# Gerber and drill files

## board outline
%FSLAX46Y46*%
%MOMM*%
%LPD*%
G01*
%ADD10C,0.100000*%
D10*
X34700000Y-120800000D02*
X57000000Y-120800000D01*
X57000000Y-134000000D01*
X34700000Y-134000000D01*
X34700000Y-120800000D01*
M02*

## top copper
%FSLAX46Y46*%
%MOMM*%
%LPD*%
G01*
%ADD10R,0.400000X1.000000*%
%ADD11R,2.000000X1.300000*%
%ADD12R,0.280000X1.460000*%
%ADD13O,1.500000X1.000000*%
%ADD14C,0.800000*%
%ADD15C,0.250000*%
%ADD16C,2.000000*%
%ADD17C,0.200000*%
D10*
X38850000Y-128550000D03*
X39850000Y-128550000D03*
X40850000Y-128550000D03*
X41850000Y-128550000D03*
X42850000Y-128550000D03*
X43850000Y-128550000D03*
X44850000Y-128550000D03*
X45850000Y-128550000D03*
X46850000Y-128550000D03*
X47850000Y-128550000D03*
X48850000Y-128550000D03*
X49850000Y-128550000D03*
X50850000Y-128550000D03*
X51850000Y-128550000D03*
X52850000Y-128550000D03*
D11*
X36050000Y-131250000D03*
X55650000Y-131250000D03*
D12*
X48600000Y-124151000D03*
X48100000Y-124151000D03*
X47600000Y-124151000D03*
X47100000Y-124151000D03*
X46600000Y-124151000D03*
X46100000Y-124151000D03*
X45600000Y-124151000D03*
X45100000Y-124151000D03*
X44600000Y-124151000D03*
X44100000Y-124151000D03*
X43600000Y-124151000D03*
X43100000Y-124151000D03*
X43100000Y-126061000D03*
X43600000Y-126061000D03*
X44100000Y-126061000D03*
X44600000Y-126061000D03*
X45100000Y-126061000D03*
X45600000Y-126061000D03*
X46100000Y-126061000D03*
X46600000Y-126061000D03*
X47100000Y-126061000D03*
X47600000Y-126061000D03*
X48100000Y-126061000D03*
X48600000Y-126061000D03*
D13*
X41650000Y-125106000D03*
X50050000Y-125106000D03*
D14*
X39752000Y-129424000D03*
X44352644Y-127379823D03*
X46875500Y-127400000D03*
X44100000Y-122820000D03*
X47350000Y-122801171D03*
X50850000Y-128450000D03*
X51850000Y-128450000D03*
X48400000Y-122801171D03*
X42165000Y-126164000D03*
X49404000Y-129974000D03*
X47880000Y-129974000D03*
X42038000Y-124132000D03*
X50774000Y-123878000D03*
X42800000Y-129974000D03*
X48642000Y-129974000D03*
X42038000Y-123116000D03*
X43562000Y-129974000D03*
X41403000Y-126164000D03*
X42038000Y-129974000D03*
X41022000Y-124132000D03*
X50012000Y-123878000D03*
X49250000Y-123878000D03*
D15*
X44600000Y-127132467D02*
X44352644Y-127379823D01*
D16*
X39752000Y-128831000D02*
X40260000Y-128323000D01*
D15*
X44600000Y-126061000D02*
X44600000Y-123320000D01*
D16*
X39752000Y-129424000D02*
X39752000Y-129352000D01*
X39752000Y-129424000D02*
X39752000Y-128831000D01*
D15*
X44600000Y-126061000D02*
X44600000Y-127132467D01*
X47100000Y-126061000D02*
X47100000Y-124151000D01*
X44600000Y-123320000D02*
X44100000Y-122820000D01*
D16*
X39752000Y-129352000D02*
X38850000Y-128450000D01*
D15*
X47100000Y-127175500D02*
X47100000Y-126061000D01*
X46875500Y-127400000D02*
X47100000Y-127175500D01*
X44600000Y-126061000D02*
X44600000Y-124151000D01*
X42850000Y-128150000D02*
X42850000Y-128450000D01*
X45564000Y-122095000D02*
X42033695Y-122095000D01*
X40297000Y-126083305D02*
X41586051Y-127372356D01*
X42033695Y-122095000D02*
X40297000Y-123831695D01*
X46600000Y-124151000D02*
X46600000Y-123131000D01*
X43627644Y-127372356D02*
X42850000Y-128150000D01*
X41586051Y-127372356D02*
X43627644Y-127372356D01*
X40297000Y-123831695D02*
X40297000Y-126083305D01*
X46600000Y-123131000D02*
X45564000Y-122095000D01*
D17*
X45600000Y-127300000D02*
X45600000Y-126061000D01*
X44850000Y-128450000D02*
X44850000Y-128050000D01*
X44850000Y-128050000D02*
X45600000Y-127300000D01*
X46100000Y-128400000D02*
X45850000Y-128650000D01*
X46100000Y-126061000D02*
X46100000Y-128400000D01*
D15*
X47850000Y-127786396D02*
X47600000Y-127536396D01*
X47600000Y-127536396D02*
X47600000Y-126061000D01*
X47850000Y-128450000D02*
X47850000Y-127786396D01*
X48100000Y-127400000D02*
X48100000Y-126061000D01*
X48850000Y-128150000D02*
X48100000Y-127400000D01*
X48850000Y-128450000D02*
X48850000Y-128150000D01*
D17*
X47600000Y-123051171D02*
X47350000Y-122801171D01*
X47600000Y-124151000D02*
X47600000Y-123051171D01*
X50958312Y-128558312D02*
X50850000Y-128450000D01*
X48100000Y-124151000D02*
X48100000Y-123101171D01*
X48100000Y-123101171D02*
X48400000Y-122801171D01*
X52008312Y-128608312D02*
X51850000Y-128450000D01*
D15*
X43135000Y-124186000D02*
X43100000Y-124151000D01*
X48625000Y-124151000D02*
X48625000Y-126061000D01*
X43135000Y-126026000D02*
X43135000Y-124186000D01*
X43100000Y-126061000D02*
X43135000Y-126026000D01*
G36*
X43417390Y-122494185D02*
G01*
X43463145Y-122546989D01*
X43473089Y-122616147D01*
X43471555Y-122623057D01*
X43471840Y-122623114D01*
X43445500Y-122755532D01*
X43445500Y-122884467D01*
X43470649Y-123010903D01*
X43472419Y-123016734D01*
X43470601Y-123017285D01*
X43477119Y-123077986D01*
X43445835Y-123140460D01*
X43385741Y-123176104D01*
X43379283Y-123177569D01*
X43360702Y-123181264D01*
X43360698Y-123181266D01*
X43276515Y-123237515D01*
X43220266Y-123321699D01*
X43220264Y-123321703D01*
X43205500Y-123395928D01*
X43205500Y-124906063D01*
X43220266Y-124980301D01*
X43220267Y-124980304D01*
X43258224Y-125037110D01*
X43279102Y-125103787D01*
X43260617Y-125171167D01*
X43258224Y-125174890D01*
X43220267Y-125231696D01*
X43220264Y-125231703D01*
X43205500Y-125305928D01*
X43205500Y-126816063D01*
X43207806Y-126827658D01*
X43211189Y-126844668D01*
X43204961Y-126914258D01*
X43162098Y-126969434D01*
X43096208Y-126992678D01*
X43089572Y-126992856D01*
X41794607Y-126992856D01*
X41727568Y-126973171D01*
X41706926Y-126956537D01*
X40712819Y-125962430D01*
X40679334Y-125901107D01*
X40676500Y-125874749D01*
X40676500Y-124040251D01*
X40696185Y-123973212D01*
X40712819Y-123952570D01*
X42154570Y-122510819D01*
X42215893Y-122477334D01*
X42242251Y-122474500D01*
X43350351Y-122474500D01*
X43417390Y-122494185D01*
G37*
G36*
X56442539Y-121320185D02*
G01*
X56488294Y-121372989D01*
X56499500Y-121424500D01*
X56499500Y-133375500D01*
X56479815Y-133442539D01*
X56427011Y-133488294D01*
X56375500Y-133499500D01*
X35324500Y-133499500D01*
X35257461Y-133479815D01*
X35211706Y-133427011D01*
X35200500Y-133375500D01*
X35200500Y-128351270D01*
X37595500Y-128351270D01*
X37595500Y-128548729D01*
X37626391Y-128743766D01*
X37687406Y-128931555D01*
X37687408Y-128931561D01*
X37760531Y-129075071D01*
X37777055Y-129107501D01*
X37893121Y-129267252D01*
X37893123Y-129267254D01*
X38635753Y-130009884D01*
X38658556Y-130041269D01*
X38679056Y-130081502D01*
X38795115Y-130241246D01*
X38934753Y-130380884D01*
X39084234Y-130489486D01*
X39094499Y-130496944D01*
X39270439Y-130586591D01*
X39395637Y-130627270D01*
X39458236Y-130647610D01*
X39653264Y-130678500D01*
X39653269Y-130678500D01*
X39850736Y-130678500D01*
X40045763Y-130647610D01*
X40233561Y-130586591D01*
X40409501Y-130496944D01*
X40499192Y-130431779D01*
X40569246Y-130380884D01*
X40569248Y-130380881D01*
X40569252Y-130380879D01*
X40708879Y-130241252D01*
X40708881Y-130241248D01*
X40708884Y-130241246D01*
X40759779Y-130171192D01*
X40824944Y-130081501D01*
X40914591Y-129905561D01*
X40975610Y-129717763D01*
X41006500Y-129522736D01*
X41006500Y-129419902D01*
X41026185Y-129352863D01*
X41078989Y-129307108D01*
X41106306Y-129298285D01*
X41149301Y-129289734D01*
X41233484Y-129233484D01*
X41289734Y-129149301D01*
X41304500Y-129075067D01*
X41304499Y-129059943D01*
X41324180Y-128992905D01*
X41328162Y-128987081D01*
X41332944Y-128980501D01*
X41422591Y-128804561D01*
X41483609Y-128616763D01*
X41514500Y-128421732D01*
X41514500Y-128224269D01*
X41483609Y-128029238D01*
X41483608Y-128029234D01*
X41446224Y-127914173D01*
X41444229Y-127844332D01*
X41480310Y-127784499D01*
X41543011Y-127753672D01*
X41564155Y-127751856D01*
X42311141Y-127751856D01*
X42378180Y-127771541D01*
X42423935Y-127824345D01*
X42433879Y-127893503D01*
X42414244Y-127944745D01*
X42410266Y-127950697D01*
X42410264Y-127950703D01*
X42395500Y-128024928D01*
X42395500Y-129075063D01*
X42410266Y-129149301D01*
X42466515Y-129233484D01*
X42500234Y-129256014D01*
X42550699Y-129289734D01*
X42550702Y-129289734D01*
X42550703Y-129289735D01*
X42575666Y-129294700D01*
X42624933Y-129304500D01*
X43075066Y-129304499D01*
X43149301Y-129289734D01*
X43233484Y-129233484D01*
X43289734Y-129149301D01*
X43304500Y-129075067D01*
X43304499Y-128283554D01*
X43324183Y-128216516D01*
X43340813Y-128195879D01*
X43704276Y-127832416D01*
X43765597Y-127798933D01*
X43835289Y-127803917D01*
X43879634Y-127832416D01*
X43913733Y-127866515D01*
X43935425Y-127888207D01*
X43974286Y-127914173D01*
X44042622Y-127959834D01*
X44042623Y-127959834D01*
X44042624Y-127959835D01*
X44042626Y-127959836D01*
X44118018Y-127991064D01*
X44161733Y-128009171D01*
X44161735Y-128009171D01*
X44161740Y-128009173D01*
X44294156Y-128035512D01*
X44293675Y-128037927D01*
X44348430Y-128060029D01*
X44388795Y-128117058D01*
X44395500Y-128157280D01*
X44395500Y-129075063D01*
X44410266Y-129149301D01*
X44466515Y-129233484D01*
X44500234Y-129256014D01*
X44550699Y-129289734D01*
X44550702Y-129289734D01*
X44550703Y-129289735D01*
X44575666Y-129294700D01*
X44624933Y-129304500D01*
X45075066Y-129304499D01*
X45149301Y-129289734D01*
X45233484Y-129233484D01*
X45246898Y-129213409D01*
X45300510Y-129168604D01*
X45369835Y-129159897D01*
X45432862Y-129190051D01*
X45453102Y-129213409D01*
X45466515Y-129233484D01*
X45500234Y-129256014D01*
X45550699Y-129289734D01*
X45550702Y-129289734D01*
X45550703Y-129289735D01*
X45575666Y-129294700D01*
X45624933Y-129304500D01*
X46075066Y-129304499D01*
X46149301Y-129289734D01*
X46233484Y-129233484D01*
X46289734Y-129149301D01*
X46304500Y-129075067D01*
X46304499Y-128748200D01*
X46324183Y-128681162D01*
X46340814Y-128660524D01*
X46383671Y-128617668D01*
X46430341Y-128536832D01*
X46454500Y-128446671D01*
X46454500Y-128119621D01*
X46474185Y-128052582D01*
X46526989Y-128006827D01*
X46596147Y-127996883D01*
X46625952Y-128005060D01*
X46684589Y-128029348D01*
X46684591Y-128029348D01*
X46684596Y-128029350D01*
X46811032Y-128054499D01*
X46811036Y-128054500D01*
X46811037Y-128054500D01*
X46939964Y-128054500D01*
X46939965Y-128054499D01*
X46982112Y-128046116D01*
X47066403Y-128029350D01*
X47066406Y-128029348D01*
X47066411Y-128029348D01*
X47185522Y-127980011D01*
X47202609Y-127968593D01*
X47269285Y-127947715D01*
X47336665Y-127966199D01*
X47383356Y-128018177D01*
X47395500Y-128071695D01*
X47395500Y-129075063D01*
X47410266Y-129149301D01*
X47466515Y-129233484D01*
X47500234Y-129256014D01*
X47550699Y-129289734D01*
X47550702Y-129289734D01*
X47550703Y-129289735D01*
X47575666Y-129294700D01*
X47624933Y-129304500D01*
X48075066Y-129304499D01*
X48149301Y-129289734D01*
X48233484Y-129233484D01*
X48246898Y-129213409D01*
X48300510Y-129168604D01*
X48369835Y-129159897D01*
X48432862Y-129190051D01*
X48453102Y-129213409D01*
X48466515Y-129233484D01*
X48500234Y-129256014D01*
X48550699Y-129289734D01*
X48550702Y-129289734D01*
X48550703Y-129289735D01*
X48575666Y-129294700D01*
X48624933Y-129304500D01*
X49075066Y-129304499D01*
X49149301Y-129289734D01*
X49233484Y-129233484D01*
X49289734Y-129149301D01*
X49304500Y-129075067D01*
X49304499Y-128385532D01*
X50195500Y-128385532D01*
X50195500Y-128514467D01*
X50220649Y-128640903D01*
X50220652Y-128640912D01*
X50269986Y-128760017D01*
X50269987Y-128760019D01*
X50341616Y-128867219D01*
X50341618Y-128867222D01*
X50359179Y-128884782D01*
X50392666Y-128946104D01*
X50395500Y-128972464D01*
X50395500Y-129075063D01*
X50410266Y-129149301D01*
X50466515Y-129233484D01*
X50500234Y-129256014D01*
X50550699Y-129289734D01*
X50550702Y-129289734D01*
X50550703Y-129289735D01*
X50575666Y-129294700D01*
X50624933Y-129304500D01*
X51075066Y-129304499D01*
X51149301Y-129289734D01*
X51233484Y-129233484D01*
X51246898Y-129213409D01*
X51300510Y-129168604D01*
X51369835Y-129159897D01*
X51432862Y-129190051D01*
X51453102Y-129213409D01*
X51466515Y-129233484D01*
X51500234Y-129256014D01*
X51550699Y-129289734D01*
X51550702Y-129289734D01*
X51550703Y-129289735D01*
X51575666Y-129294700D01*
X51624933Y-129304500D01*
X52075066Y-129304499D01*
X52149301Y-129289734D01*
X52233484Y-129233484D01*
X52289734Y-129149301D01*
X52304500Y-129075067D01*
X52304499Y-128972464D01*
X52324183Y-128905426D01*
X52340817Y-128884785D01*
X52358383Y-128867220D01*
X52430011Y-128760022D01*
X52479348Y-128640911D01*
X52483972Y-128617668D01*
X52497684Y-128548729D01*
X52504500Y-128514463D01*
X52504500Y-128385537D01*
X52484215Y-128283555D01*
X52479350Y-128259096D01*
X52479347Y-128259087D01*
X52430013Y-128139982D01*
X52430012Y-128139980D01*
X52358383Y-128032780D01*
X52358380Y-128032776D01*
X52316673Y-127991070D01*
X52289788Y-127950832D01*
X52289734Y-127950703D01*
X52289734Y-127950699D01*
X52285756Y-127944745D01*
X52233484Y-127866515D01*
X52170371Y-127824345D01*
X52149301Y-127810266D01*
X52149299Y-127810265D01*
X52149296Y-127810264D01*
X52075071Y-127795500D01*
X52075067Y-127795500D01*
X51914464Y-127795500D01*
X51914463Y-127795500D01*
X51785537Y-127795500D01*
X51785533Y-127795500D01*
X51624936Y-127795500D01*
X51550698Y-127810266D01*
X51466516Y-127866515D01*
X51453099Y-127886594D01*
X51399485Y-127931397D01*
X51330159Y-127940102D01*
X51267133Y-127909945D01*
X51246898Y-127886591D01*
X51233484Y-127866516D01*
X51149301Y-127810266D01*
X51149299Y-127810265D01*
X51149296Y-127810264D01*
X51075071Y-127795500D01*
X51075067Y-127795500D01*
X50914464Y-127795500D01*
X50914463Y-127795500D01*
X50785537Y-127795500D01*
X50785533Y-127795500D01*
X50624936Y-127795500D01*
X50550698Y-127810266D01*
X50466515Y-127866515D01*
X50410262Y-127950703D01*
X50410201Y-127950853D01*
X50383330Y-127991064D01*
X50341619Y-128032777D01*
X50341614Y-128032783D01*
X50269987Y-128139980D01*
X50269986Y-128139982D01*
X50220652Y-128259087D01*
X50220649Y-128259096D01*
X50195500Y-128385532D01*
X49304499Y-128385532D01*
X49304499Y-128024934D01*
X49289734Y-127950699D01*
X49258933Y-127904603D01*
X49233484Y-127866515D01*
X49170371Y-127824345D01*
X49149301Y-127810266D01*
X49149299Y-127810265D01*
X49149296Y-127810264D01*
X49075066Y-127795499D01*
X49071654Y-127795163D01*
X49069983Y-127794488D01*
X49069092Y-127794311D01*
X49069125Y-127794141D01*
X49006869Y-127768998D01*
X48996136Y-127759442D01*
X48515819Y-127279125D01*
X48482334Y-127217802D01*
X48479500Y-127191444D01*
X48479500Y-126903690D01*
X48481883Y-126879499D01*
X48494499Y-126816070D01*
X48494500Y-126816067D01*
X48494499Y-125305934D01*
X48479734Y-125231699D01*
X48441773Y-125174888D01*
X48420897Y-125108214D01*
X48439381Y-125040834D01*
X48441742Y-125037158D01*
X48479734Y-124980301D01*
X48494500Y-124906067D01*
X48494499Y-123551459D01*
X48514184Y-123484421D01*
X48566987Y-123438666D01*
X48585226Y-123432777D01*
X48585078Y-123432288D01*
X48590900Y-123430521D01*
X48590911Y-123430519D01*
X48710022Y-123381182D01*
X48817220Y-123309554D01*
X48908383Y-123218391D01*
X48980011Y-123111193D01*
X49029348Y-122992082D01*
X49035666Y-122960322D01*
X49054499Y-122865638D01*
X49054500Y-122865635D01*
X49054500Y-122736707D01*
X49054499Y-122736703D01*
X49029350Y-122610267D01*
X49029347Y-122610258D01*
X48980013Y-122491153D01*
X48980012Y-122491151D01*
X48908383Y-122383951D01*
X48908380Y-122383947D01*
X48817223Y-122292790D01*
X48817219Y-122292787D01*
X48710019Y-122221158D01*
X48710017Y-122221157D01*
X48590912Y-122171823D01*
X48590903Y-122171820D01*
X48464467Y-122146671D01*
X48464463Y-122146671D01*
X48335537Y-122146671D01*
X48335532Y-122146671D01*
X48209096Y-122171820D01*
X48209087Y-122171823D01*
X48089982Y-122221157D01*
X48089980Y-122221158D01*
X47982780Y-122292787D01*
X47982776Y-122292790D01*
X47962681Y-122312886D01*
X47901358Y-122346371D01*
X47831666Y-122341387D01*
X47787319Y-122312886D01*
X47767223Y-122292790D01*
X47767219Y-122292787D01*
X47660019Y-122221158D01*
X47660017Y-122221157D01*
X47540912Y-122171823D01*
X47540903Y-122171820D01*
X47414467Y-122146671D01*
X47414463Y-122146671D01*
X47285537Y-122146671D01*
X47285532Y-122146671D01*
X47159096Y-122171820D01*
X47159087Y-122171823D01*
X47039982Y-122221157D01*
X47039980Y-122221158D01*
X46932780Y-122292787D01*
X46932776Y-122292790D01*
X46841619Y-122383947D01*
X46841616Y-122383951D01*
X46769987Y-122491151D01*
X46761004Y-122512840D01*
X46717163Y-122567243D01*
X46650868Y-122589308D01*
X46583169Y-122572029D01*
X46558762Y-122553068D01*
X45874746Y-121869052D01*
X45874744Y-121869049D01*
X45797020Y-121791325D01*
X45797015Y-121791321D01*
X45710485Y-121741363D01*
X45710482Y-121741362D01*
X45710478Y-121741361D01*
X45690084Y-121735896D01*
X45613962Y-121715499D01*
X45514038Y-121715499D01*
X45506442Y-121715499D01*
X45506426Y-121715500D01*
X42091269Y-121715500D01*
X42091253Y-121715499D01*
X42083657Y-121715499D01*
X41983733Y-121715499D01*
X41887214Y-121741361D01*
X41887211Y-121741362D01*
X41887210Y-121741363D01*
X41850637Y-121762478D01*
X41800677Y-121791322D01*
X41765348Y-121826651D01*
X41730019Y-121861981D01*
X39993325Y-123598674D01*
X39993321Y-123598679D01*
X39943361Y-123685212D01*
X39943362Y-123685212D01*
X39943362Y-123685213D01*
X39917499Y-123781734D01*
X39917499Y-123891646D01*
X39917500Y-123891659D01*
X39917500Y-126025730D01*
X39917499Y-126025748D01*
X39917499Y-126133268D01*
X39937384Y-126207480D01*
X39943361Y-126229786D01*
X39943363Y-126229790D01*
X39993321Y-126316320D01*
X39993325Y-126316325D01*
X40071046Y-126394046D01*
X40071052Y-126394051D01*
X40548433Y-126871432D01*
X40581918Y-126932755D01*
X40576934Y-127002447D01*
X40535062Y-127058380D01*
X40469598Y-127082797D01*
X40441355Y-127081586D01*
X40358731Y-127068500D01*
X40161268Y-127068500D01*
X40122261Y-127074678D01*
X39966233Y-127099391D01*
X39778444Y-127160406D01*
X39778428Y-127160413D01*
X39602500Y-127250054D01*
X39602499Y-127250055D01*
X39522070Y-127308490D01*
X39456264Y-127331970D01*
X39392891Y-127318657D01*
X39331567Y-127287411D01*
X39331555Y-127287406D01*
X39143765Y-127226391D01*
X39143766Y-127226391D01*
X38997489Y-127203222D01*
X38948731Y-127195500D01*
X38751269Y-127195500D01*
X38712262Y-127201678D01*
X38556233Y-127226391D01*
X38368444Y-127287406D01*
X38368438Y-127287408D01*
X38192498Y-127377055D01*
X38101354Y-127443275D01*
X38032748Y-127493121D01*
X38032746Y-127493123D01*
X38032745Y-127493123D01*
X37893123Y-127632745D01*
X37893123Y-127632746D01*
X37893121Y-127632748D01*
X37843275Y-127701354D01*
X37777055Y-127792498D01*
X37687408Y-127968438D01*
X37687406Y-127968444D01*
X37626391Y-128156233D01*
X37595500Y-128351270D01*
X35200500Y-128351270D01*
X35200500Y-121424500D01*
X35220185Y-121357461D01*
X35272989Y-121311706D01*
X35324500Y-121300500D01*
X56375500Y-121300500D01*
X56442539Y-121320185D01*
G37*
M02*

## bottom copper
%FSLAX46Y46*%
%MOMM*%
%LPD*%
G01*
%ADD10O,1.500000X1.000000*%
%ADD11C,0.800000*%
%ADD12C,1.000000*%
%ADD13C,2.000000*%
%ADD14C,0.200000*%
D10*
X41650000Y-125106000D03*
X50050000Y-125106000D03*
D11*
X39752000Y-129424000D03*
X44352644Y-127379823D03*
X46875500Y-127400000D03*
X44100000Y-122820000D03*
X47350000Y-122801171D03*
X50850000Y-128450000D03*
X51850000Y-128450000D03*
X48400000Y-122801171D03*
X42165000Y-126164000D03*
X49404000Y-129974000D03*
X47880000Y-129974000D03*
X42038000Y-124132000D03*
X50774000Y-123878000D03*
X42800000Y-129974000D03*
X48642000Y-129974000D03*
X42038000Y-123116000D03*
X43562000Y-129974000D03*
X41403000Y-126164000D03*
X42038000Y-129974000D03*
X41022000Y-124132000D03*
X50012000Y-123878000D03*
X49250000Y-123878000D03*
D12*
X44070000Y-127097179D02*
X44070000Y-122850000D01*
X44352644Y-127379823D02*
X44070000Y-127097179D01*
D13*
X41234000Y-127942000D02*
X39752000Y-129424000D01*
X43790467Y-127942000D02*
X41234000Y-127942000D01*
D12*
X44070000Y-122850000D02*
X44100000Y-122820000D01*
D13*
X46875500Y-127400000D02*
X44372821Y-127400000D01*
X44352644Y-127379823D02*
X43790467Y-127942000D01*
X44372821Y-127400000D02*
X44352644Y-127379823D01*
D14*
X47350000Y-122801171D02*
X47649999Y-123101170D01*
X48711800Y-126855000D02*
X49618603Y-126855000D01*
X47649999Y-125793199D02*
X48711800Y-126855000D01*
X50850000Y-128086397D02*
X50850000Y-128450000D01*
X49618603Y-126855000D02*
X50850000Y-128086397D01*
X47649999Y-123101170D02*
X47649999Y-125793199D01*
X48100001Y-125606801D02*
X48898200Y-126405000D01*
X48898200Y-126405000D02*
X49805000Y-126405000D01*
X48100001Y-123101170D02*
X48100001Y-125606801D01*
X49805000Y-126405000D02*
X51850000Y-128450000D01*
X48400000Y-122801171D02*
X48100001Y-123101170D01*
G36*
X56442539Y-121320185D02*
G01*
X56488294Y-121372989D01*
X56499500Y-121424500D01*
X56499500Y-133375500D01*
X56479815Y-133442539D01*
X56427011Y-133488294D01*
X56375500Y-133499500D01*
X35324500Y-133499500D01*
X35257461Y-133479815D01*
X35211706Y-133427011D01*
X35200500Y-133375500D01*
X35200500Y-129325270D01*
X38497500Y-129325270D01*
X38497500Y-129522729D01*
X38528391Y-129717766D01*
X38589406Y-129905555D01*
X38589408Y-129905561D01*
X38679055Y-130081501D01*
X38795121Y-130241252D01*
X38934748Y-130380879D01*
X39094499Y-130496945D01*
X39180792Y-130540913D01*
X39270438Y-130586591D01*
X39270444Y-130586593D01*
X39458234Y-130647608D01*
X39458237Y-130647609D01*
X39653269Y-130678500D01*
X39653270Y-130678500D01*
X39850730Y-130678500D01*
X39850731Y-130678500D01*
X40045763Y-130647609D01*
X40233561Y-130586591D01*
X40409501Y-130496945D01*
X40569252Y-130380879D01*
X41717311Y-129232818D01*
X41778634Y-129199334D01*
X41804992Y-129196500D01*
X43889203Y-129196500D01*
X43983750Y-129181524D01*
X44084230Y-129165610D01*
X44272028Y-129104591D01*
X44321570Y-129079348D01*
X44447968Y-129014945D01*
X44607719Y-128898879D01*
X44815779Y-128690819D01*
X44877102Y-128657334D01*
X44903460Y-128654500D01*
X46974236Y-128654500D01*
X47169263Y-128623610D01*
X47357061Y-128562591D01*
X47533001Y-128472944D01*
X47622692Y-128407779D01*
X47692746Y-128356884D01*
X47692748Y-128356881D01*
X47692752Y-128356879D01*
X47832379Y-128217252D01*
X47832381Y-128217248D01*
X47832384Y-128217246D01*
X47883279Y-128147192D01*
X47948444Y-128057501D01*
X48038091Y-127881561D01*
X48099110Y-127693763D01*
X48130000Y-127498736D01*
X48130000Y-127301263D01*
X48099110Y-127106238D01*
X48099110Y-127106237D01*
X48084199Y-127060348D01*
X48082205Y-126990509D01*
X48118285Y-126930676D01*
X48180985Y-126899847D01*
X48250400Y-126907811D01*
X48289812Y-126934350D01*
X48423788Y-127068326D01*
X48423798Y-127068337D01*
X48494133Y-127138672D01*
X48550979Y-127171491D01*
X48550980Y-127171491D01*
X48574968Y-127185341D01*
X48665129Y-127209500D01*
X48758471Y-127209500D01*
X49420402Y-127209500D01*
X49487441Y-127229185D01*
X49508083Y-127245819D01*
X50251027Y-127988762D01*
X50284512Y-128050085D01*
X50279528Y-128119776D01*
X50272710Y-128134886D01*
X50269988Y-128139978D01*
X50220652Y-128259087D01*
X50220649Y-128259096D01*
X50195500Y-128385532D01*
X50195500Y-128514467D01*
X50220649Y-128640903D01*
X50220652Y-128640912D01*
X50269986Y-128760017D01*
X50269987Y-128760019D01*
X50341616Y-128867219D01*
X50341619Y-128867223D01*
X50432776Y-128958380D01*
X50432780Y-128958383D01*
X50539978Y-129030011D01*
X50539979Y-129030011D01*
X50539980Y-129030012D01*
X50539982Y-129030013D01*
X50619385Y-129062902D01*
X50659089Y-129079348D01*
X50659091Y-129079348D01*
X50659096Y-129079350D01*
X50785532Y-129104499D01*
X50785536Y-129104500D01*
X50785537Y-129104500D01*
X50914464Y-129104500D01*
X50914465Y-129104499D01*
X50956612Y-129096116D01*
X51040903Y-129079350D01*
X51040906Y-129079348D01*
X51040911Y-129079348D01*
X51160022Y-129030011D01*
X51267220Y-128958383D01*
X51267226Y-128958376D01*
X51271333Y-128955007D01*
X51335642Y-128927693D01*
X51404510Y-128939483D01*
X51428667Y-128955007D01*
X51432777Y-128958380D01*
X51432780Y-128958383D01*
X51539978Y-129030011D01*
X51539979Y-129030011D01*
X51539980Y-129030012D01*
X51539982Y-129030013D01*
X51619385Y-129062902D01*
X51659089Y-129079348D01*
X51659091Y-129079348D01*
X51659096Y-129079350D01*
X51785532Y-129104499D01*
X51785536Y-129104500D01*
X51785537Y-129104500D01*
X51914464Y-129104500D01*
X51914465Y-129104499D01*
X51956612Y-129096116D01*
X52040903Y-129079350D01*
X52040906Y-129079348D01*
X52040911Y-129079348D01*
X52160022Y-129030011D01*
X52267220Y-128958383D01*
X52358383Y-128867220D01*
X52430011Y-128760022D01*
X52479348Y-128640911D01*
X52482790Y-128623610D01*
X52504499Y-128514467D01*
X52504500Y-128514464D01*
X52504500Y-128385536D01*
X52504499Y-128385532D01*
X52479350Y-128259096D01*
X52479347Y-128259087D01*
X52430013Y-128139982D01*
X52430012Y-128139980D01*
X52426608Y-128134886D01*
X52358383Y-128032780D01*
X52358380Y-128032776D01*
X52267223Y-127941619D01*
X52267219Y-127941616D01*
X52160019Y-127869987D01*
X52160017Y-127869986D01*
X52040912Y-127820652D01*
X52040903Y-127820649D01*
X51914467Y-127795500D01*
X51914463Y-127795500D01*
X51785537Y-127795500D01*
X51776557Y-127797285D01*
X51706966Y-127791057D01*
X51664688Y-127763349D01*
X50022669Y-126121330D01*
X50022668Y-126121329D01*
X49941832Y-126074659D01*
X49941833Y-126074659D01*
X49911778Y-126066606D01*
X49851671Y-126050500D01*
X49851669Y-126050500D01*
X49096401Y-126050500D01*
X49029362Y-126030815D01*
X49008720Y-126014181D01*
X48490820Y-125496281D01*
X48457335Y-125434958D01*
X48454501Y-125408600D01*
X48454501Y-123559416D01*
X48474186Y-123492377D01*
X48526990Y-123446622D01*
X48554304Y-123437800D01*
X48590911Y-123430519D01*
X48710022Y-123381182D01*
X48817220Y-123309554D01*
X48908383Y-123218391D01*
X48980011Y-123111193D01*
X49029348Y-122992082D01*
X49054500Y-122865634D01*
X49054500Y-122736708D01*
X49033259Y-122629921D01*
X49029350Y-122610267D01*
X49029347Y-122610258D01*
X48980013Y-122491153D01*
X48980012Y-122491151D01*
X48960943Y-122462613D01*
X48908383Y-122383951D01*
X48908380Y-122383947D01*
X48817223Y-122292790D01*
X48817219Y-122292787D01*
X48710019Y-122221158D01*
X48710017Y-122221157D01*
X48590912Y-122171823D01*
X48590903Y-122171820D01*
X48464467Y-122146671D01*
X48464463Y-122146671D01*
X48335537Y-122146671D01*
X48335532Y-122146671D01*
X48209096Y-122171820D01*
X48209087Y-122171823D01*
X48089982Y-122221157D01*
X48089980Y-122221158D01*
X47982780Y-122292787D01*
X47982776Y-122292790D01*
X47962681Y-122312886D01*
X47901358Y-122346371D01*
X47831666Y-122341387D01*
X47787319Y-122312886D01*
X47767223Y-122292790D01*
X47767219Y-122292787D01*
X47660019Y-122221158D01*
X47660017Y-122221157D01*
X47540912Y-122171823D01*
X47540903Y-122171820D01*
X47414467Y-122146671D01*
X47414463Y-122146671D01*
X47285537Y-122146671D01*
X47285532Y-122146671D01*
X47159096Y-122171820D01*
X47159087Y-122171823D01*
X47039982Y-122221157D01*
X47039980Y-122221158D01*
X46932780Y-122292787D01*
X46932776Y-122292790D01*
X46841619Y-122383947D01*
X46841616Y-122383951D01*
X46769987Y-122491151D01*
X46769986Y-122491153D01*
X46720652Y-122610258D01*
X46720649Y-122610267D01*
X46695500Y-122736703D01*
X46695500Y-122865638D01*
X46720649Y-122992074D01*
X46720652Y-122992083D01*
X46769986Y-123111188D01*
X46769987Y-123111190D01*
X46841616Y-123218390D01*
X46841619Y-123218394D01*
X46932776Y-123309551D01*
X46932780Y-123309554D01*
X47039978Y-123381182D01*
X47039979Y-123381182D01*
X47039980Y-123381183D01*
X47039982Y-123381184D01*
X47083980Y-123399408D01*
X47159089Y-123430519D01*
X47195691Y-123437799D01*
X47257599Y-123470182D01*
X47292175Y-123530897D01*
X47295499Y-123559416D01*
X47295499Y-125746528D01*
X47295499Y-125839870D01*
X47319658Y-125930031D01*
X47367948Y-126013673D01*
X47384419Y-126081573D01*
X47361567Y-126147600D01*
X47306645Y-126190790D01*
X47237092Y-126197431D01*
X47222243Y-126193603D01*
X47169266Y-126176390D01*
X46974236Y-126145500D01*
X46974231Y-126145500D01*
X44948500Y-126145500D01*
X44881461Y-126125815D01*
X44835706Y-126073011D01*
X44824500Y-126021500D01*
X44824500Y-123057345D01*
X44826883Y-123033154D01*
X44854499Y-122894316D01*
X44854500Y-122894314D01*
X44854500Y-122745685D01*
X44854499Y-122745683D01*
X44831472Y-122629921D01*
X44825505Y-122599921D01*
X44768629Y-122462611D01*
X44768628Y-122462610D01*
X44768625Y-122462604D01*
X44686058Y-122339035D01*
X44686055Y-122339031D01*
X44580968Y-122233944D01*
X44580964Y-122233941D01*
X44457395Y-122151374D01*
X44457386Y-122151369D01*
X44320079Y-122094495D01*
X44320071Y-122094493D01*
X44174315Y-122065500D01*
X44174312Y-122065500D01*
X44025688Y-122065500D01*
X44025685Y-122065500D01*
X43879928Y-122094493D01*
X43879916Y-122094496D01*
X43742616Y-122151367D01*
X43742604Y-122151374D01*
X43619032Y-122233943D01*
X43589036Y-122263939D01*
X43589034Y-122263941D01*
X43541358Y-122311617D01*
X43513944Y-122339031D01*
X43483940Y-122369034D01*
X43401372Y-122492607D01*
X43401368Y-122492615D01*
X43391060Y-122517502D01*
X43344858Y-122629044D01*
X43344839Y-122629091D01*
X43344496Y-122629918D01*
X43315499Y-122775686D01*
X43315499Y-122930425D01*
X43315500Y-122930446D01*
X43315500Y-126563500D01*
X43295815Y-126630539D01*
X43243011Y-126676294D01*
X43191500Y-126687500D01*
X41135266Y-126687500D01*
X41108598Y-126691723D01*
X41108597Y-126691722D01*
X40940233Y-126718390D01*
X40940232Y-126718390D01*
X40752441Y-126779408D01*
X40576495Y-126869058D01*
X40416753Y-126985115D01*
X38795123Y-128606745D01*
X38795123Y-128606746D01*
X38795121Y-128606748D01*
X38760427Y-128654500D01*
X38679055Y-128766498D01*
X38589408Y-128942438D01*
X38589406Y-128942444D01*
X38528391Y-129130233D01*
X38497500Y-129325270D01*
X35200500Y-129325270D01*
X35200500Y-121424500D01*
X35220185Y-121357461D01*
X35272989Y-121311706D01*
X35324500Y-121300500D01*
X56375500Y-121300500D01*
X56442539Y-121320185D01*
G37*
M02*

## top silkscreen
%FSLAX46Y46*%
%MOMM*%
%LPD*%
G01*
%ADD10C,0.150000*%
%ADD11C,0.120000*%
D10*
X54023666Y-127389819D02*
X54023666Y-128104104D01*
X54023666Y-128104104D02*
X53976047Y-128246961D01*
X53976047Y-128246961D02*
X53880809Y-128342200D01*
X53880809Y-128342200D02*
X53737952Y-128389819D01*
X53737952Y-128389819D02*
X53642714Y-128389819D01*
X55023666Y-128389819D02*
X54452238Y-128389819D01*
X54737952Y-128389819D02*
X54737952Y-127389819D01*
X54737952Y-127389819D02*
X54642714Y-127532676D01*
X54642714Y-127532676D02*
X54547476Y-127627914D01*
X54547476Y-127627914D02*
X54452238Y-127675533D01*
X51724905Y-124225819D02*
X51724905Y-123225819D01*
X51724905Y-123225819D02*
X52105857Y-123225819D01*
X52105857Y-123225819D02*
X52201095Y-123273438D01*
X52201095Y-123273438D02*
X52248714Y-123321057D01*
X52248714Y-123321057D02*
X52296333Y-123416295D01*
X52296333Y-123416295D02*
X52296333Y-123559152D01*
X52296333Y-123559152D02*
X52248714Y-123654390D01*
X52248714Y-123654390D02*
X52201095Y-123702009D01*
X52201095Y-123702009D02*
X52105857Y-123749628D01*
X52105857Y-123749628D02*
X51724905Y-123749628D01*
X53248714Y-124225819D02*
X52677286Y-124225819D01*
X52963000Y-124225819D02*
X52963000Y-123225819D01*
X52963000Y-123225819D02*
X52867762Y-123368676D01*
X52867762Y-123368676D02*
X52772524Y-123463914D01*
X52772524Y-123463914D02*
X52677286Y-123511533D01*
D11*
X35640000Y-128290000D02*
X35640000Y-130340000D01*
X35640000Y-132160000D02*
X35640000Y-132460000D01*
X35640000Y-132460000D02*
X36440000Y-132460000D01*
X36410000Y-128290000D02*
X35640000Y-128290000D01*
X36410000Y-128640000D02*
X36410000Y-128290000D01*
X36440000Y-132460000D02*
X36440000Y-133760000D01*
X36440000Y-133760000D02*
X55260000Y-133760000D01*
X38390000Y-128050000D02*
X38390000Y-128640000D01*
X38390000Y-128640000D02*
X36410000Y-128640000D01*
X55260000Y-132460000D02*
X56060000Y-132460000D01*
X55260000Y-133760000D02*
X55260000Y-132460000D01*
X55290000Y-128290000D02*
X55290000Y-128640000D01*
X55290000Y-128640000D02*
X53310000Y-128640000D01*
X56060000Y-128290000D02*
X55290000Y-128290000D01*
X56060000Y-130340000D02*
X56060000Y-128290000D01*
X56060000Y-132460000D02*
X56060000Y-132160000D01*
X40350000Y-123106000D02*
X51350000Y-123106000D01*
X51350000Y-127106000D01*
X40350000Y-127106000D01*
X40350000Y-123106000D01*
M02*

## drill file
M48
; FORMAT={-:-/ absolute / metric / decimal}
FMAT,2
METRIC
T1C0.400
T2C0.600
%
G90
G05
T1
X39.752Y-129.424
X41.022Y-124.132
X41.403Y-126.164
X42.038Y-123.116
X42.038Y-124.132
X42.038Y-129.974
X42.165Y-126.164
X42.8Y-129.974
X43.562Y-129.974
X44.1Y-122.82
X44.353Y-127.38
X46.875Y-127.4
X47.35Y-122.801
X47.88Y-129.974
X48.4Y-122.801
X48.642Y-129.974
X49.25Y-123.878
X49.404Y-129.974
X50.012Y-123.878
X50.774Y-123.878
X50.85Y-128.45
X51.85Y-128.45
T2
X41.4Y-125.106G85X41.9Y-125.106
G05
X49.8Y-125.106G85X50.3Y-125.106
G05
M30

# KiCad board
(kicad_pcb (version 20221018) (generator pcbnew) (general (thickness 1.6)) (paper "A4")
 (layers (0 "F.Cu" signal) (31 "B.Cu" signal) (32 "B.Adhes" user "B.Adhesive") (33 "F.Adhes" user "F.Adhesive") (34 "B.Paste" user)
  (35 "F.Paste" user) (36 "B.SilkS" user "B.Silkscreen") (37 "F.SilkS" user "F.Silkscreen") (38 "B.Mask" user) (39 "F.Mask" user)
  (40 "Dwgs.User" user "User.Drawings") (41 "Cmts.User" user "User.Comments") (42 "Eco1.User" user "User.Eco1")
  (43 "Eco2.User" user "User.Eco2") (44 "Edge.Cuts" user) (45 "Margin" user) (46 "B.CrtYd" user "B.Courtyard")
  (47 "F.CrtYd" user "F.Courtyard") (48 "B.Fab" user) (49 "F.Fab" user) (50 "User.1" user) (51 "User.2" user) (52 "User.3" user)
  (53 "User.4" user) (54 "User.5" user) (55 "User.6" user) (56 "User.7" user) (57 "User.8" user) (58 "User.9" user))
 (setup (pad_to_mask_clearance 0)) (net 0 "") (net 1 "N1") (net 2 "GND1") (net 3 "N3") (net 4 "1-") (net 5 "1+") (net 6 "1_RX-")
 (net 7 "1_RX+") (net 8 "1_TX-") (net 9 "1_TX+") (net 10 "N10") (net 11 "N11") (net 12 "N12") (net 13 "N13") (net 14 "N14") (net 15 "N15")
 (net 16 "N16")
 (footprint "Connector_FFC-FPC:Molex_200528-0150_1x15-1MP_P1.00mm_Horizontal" (layer "F.Cu") (at 45.85 129.46)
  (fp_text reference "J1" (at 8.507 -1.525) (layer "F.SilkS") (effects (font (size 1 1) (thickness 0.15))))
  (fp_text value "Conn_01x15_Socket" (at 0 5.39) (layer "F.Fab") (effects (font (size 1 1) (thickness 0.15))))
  (fp_line (start -10.21 -1.17) (end -10.21 0.88) (stroke (width 0.12) (type solid)) (layer "F.SilkS"))
  (fp_line (start -10.21 2.7) (end -10.21 3) (stroke (width 0.12) (type solid)) (layer "F.SilkS"))
  (fp_line (start -10.21 3) (end -9.41 3) (stroke (width 0.12) (type solid)) (layer "F.SilkS"))
  (fp_line (start -9.44 -1.17) (end -10.21 -1.17) (stroke (width 0.12) (type solid)) (layer "F.SilkS"))
  (fp_line (start -9.44 -0.82) (end -9.44 -1.17) (stroke (width 0.12) (type solid)) (layer "F.SilkS"))
  (fp_line (start -9.41 3) (end -9.41 4.3) (stroke (width 0.12) (type solid)) (layer "F.SilkS"))
  (fp_line (start -9.41 4.3) (end 9.41 4.3) (stroke (width 0.12) (type solid)) (layer "F.SilkS"))
  (fp_line (start -7.46 -1.41) (end -7.46 -0.82) (stroke (width 0.12) (type solid)) (layer "F.SilkS"))
  (fp_line (start -7.46 -0.82) (end -9.44 -0.82) (stroke (width 0.12) (type solid)) (layer "F.SilkS"))
  (fp_line (start 9.41 3) (end 10.21 3) (stroke (width 0.12) (type solid)) (layer "F.SilkS"))
  (fp_line (start 9.41 4.3) (end 9.41 3) (stroke (width 0.12) (type solid)) (layer "F.SilkS"))
  (fp_line (start 9.44 -1.17) (end 9.44 -0.82) (stroke (width 0.12) (type solid)) (layer "F.SilkS"))
  (fp_line (start 9.44 -0.82) (end 7.46 -0.82) (stroke (width 0.12) (type solid)) (layer "F.SilkS"))
  (fp_line (start 10.21 -1.17) (end 9.44 -1.17) (stroke (width 0.12) (type solid)) (layer "F.SilkS"))
  (fp_line (start 10.21 0.88) (end 10.21 -1.17) (stroke (width 0.12) (type solid)) (layer "F.SilkS"))
  (fp_line (start 10.21 3) (end 10.21 2.7) (stroke (width 0.12) (type solid)) (layer "F.SilkS"))
  (pad "1" smd rect (at -7 -0.91) (size 0.4 1) (layers "F.Cu" "F.Paste" "F.Mask") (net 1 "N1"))
  (pad "2" smd rect (at -6 -0.91) (size 0.4 1) (layers "F.Cu" "F.Paste" "F.Mask") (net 1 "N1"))
  (pad "3" smd rect (at -5 -0.91) (size 0.4 1) (layers "F.Cu" "F.Paste" "F.Mask") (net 1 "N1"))
  (pad "4" smd rect (at -4 -0.91) (size 0.4 1) (layers "F.Cu" "F.Paste" "F.Mask") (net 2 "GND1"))
  (pad "5" smd rect (at -3 -0.91) (size 0.4 1) (layers "F.Cu" "F.Paste" "F.Mask") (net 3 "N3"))
  (pad "6" smd rect (at -2 -0.91) (size 0.4 1) (layers "F.Cu" "F.Paste" "F.Mask") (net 2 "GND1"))
  (pad "7" smd rect (at -1 -0.91) (size 0.4 1) (layers "F.Cu" "F.Paste" "F.Mask") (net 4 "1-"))
  (pad "8" smd rect (at 0 -0.91) (size 0.4 1) (layers "F.Cu" "F.Paste" "F.Mask") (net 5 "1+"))
  (pad "9" smd rect (at 1 -0.91) (size 0.4 1) (layers "F.Cu" "F.Paste" "F.Mask") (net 2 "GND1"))
  (pad "10" smd rect (at 2 -0.91) (size 0.4 1) (layers "F.Cu" "F.Paste" "F.Mask") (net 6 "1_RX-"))
  (pad "11" smd rect (at 3 -0.91) (size 0.4 1) (layers "F.Cu" "F.Paste" "F.Mask") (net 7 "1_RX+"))
  (pad "12" smd rect (at 4 -0.91) (size 0.4 1) (layers "F.Cu" "F.Paste" "F.Mask") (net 2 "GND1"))
  (pad "13" smd rect (at 5 -0.91) (size 0.4 1) (layers "F.Cu" "F.Paste" "F.Mask") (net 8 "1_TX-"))
  (pad "14" smd rect (at 6 -0.91) (size 0.4 1) (layers "F.Cu" "F.Paste" "F.Mask") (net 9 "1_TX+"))
  (pad "15" smd rect (at 7 -0.91) (size 0.4 1) (layers "F.Cu" "F.Paste" "F.Mask") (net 2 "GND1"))
  (pad "MP" smd rect (at -9.8 1.79) (size 2 1.3) (layers "F.Cu" "F.Paste" "F.Mask") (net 2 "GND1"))
  (pad "MP" smd rect (at 9.8 1.79) (size 2 1.3) (layers "F.Cu" "F.Paste" "F.Mask") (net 2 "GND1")))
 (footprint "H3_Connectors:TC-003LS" (layer "F.Cu") (at 45.85 125.106)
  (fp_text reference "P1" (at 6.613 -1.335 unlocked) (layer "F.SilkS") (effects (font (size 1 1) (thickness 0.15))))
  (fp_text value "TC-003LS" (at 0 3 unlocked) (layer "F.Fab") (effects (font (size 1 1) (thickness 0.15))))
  (fp_rect (start -5.5 -2) (end 5.5 2) (stroke (width 0.12) (type default)) (fill none) (layer "F.SilkS"))
  (pad "A1" smd rect (at 2.75 -0.955) (size 0.28 1.46) (layers "F.Cu" "F.Paste" "F.Mask") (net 2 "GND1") (thermal_bridge_angle 45))
  (pad "A2" smd rect (at 2.25 -0.955) (size 0.28 1.46) (layers "F.Cu" "F.Paste" "F.Mask") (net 9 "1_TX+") (thermal_bridge_angle 45))
  (pad "A3" smd rect (at 1.75 -0.955) (size 0.28 1.46) (layers "F.Cu" "F.Paste" "F.Mask") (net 8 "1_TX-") (thermal_bridge_angle 45))
  (pad "A4" smd rect (at 1.25 -0.955) (size 0.28 1.46) (layers "F.Cu" "F.Paste" "F.Mask") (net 1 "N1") (thermal_bridge_angle 45))
  (pad "A5" smd rect (at 0.75 -0.955) (size 0.28 1.46) (layers "F.Cu" "F.Paste" "F.Mask") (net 3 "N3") (thermal_bridge_angle 45))
  (pad "A6" smd rect (at 0.25 -0.955) (size 0.28 1.46) (layers "F.Cu" "F.Paste" "F.Mask") (thermal_bridge_angle 45))
  (pad "A7" smd rect (at -0.25 -0.955) (size 0.28 1.46) (layers "F.Cu" "F.Paste" "F.Mask") (thermal_bridge_angle 45))
  (pad "A8" smd rect (at -0.75 -0.955) (size 0.28 1.46) (layers "F.Cu" "F.Paste" "F.Mask") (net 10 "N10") (thermal_bridge_angle 45))
  (pad "A9" smd rect (at -1.25 -0.955) (size 0.28 1.46) (layers "F.Cu" "F.Paste" "F.Mask") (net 1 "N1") (thermal_bridge_angle 45))
  (pad "A10" smd rect (at -1.75 -0.955) (size 0.28 1.46) (layers "F.Cu" "F.Paste" "F.Mask") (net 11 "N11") (thermal_bridge_angle 45))
  (pad "A11" smd rect (at -2.25 -0.955) (size 0.28 1.46) (layers "F.Cu" "F.Paste" "F.Mask") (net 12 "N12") (thermal_bridge_angle 45))
  (pad "A12" smd rect (at -2.75 -0.955) (size 0.28 1.46) (layers "F.Cu" "F.Paste" "F.Mask") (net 2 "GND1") (thermal_bridge_angle 45))
  (pad "B1" smd rect (at -2.75 0.955 180) (size 0.28 1.46) (layers "F.Cu" "F.Paste" "F.Mask") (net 2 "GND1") (thermal_bridge_angle 45))
  (pad "B2" smd rect (at -2.25 0.955 180) (size 0.28 1.46) (layers "F.Cu" "F.Paste" "F.Mask") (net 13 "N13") (thermal_bridge_angle 45))
  (pad "B3" smd rect (at -1.75 0.955 180) (size 0.28 1.46) (layers "F.Cu" "F.Paste" "F.Mask") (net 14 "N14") (thermal_bridge_angle 45))
  (pad "B4" smd rect (at -1.25 0.955 180) (size 0.28 1.46) (layers "F.Cu" "F.Paste" "F.Mask") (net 1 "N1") (thermal_bridge_angle 45))
  (pad "B5" smd rect (at -0.75 0.955 180) (size 0.28 1.46) (layers "F.Cu" "F.Paste" "F.Mask") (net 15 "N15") (thermal_bridge_angle 45))
  (pad "B6" smd rect (at -0.25 0.955 180) (size 0.28 1.46) (layers "F.Cu" "F.Paste" "F.Mask") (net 4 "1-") (thermal_bridge_angle 45))
  (pad "B7" smd rect (at 0.25 0.955 180) (size 0.28 1.46) (layers "F.Cu" "F.Paste" "F.Mask") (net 5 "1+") (thermal_bridge_angle 45))
  (pad "B8" smd rect (at 0.75 0.955 180) (size 0.28 1.46) (layers "F.Cu" "F.Paste" "F.Mask") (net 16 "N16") (thermal_bridge_angle 45))
  (pad "B9" smd rect (at 1.25 0.955 180) (size 0.28 1.46) (layers "F.Cu" "F.Paste" "F.Mask") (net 1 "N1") (thermal_bridge_angle 45))
  (pad "B10" smd rect (at 1.75 0.955 180) (size 0.28 1.46) (layers "F.Cu" "F.Paste" "F.Mask") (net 6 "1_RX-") (thermal_bridge_angle 45))
  (pad "B11" smd rect (at 2.25 0.955 180) (size 0.28 1.46) (layers "F.Cu" "F.Paste" "F.Mask") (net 7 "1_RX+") (thermal_bridge_angle 45))
  (pad "B12" smd rect (at 2.75 0.955 180) (size 0.28 1.46) (layers "F.Cu" "F.Paste" "F.Mask") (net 2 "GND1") (thermal_bridge_angle 45))
  (pad "S1" thru_hole oval (at -4.2 0) (size 1.5 1) (drill oval 1.1 0.6) (layers "*.Cu" "*.Mask") (remove_unused_layers) (keep_end_layers)
   (zone_layer_connections) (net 2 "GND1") (thermal_bridge_angle 45))
  (pad "S1" thru_hole oval (at 4.2 0) (size 1.5 1) (drill oval 1.1 0.6) (layers "*.Cu" "*.Mask") (remove_unused_layers) (keep_end_layers)
   (zone_layer_connections) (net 2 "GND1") (thermal_bridge_angle 45)))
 (gr_rect (start 34.7 120.8) (end 57 134) (stroke (width 0.1) (type default)) (fill none) (layer "Edge.Cuts"))
 (segment (start 44.6 127.132467) (end 44.352644 127.379823) (width 0.25) (layer "F.Cu") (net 1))
 (segment (start 39.752 128.831) (end 40.26 128.323) (width 2) (layer "F.Cu") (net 1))
 (segment (start 44.6 126.061) (end 44.6 123.32) (width 0.25) (layer "F.Cu") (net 1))
 (segment (start 39.752 129.424) (end 39.752 129.352) (width 2) (layer "F.Cu") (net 1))
 (segment (start 39.752 129.424) (end 39.752 128.831) (width 2) (layer "F.Cu") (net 1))
 (segment (start 44.6 126.061) (end 44.6 127.132467) (width 0.25) (layer "F.Cu") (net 1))
 (segment (start 47.1 126.061) (end 47.1 124.151) (width 0.25) (layer "F.Cu") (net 1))
 (segment (start 44.6 123.32) (end 44.1 122.82) (width 0.25) (layer "F.Cu") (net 1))
 (segment (start 39.752 129.352) (end 38.85 128.45) (width 2) (layer "F.Cu") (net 1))
 (segment (start 47.1 127.1755) (end 47.1 126.061) (width 0.25) (layer "F.Cu") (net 1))
 (segment (start 46.8755 127.4) (end 47.1 127.1755) (width 0.25) (layer "F.Cu") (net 1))
 (segment (start 44.6 126.061) (end 44.6 124.151) (width 0.25) (layer "F.Cu") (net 1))
 (via (at 39.752 129.424) (size 0.8) (drill 0.4) (layers "F.Cu" "B.Cu") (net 1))
 (via (at 44.352644 127.379823) (size 0.8) (drill 0.4) (layers "F.Cu" "B.Cu") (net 1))
 (via (at 46.8755 127.4) (size 0.8) (drill 0.4) (layers "F.Cu" "B.Cu") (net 1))
 (via (at 44.1 122.82) (size 0.8) (drill 0.4) (layers "F.Cu" "B.Cu") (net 1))
 (segment (start 44.07 127.097179) (end 44.07 122.85) (width 1) (layer "B.Cu") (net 1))
 (segment (start 44.352644 127.379823) (end 44.07 127.097179) (width 1) (layer "B.Cu") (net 1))
 (segment (start 41.234 127.942) (end 39.752 129.424) (width 2) (layer "B.Cu") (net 1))
 (segment (start 43.790467 127.942) (end 41.234 127.942) (width 2) (layer "B.Cu") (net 1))
 (segment (start 44.07 122.85) (end 44.1 122.82) (width 1) (layer "B.Cu") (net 1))
 (segment (start 46.8755 127.4) (end 44.372821 127.4) (width 2) (layer "B.Cu") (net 1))
 (segment (start 44.352644 127.379823) (end 43.790467 127.942) (width 2) (layer "B.Cu") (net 1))
 (segment (start 44.372821 127.4) (end 44.352644 127.379823) (width 2) (layer "B.Cu") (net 1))
 (segment (start 42.85 128.15) (end 42.85 128.45) (width 0.25) (layer "F.Cu") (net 3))
 (segment (start 45.564 122.095) (end 42.033695 122.095) (width 0.25) (layer "F.Cu") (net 3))
 (segment (start 40.297 126.083305) (end 41.586051 127.372356) (width 0.25) (layer "F.Cu") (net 3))
 (segment (start 42.033695 122.095) (end 40.297 123.831695) (width 0.25) (layer "F.Cu") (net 3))
 (segment (start 46.6 124.151) (end 46.6 123.131) (width 0.25) (layer "F.Cu") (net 3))
 (segment (start 43.627644 127.372356) (end 42.85 128.15) (width 0.25) (layer "F.Cu") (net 3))
 (segment (start 41.586051 127.372356) (end 43.627644 127.372356) (width 0.25) (layer "F.Cu") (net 3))
 (segment (start 40.297 123.831695) (end 40.297 126.083305) (width 0.25) (layer "F.Cu") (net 3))
 (segment (start 46.6 123.131) (end 45.564 122.095) (width 0.25) (layer "F.Cu") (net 3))
 (segment (start 45.6 127.3) (end 45.6 126.061) (width 0.2) (layer "F.Cu") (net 4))
 (segment (start 44.85 128.45) (end 44.85 128.05) (width 0.2) (layer "F.Cu") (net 4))
 (segment (start 44.85 128.05) (end 45.6 127.3) (width 0.2) (layer "F.Cu") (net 4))
 (segment (start 46.1 128.4) (end 45.85 128.65) (width 0.2) (layer "F.Cu") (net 5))
 (segment (start 46.1 126.061) (end 46.1 128.4) (width 0.2) (layer "F.Cu") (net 5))
 (segment (start 47.85 127.786396) (end 47.6 127.536396) (width 0.25) (layer "F.Cu") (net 6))
 (segment (start 47.6 127.536396) (end 47.6 126.061) (width 0.25) (layer "F.Cu") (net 6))
 (segment (start 47.85 128.45) (end 47.85 127.786396) (width 0.25) (layer "F.Cu") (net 6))
 (segment (start 48.1 127.4) (end 48.1 126.061) (width 0.25) (layer "F.Cu") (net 7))
 (segment (start 48.85 128.15) (end 48.1 127.4) (width 0.25) (layer "F.Cu") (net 7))
 (segment (start 48.85 128.45) (end 48.85 128.15) (width 0.25) (layer "F.Cu") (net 7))
 (segment (start 47.6 123.051171) (end 47.35 122.801171) (width 0.2) (layer "F.Cu") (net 8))
 (segment (start 47.6 124.151) (end 47.6 123.051171) (width 0.2) (layer "F.Cu") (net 8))
 (segment (start 50.958312 128.558312) (end 50.85 128.45) (width 0.2) (layer "F.Cu") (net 8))
 (via (at 47.35 122.801171) (size 0.8) (drill 0.4) (layers "F.Cu" "B.Cu") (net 8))
 (via (at 50.85 128.45) (size 0.8) (drill 0.4) (layers "F.Cu" "B.Cu") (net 8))
 (segment (start 47.35 122.801171) (end 47.649999 123.10117) (width 0.2) (layer "B.Cu") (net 8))
 (segment (start 48.7118 126.855) (end 49.618603 126.855) (width 0.2) (layer "B.Cu") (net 8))
 (segment (start 47.649999 125.793199) (end 48.7118 126.855) (width 0.2) (layer "B.Cu") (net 8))
 (segment (start 50.85 128.086397) (end 50.85 128.45) (width 0.2) (layer "B.Cu") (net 8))
 (segment (start 49.618603 126.855) (end 50.85 128.086397) (width 0.2) (layer "B.Cu") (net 8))
 (segment (start 47.649999 123.10117) (end 47.649999 125.793199) (width 0.2) (layer "B.Cu") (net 8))
 (segment (start 48.1 124.151) (end 48.1 123.101171) (width 0.2) (layer "F.Cu") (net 9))
 (segment (start 48.1 123.101171) (end 48.4 122.801171) (width 0.2) (layer "F.Cu") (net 9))
 (segment (start 52.008312 128.608312) (end 51.85 128.45) (width 0.2) (layer "F.Cu") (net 9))
 (via (at 51.85 128.45) (size 0.8) (drill 0.4) (layers "F.Cu" "B.Cu") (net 9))
 (via (at 48.4 122.801171) (size 0.8) (drill 0.4) (layers "F.Cu" "B.Cu") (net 9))
 (segment (start 48.100001 125.606801) (end 48.8982 126.405) (width 0.2) (layer "B.Cu") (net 9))
 (segment (start 48.8982 126.405) (end 49.805 126.405) (width 0.2) (layer "B.Cu") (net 9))
 (segment (start 48.100001 123.10117) (end 48.100001 125.606801) (width 0.2) (layer "B.Cu") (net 9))
 (segment (start 49.805 126.405) (end 51.85 128.45) (width 0.2) (layer "B.Cu") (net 9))
 (segment (start 48.4 122.801171) (end 48.100001 123.10117) (width 0.2) (layer "B.Cu") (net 9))
 (segment (start 43.135 124.186) (end 43.1 124.151) (width 0.25) (layer "F.Cu") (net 2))
 (segment (start 48.625 124.151) (end 48.625 126.061) (width 0.25) (layer "F.Cu") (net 2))
 (segment (start 43.135 126.026) (end 43.135 124.186) (width 0.25) (layer "F.Cu") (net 2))
 (segment (start 43.1 126.061) (end 43.135 126.026) (width 0.25) (layer "F.Cu") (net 2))
 (via (at 42.165 126.164) (size 0.8) (drill 0.4) (layers "F.Cu" "B.Cu") (free) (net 2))
 (via (at 49.404 129.974) (size 0.8) (drill 0.4) (layers "F.Cu" "B.Cu") (free) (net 2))
 (via (at 47.88 129.974) (size 0.8) (drill 0.4) (layers "F.Cu" "B.Cu") (free) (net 2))
 (via (at 42.038 124.132) (size 0.8) (drill 0.4) (layers "F.Cu" "B.Cu") (free) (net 2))
 (via (at 50.774 123.878) (size 0.8) (drill 0.4) (layers "F.Cu" "B.Cu") (free) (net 2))
 (via (at 42.8 129.974) (size 0.8) (drill 0.4) (layers "F.Cu" "B.Cu") (free) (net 2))
 (via (at 48.642 129.974) (size 0.8) (drill 0.4) (layers "F.Cu" "B.Cu") (free) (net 2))
 (via (at 42.038 123.116) (size 0.8) (drill 0.4) (layers "F.Cu" "B.Cu") (free) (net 2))
 (via (at 43.562 129.974) (size 0.8) (drill 0.4) (layers "F.Cu" "B.Cu") (free) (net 2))
 (via (at 41.403 126.164) (size 0.8) (drill 0.4) (layers "F.Cu" "B.Cu") (free) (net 2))
 (via (at 42.038 129.974) (size 0.8) (drill 0.4) (layers "F.Cu" "B.Cu") (free) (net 2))
 (via (at 41.022 124.132) (size 0.8) (drill 0.4) (layers "F.Cu" "B.Cu") (free) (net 2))
 (via (at 50.012 123.878) (size 0.8) (drill 0.4) (layers "F.Cu" "B.Cu") (free) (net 2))
 (via (at 49.25 123.878) (size 0.8) (drill 0.4) (layers "F.Cu" "B.Cu") (free) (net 2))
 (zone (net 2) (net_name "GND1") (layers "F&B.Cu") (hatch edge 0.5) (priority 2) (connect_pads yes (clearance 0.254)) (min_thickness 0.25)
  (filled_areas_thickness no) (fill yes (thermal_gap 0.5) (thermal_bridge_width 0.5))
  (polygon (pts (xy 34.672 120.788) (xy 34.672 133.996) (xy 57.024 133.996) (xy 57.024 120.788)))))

